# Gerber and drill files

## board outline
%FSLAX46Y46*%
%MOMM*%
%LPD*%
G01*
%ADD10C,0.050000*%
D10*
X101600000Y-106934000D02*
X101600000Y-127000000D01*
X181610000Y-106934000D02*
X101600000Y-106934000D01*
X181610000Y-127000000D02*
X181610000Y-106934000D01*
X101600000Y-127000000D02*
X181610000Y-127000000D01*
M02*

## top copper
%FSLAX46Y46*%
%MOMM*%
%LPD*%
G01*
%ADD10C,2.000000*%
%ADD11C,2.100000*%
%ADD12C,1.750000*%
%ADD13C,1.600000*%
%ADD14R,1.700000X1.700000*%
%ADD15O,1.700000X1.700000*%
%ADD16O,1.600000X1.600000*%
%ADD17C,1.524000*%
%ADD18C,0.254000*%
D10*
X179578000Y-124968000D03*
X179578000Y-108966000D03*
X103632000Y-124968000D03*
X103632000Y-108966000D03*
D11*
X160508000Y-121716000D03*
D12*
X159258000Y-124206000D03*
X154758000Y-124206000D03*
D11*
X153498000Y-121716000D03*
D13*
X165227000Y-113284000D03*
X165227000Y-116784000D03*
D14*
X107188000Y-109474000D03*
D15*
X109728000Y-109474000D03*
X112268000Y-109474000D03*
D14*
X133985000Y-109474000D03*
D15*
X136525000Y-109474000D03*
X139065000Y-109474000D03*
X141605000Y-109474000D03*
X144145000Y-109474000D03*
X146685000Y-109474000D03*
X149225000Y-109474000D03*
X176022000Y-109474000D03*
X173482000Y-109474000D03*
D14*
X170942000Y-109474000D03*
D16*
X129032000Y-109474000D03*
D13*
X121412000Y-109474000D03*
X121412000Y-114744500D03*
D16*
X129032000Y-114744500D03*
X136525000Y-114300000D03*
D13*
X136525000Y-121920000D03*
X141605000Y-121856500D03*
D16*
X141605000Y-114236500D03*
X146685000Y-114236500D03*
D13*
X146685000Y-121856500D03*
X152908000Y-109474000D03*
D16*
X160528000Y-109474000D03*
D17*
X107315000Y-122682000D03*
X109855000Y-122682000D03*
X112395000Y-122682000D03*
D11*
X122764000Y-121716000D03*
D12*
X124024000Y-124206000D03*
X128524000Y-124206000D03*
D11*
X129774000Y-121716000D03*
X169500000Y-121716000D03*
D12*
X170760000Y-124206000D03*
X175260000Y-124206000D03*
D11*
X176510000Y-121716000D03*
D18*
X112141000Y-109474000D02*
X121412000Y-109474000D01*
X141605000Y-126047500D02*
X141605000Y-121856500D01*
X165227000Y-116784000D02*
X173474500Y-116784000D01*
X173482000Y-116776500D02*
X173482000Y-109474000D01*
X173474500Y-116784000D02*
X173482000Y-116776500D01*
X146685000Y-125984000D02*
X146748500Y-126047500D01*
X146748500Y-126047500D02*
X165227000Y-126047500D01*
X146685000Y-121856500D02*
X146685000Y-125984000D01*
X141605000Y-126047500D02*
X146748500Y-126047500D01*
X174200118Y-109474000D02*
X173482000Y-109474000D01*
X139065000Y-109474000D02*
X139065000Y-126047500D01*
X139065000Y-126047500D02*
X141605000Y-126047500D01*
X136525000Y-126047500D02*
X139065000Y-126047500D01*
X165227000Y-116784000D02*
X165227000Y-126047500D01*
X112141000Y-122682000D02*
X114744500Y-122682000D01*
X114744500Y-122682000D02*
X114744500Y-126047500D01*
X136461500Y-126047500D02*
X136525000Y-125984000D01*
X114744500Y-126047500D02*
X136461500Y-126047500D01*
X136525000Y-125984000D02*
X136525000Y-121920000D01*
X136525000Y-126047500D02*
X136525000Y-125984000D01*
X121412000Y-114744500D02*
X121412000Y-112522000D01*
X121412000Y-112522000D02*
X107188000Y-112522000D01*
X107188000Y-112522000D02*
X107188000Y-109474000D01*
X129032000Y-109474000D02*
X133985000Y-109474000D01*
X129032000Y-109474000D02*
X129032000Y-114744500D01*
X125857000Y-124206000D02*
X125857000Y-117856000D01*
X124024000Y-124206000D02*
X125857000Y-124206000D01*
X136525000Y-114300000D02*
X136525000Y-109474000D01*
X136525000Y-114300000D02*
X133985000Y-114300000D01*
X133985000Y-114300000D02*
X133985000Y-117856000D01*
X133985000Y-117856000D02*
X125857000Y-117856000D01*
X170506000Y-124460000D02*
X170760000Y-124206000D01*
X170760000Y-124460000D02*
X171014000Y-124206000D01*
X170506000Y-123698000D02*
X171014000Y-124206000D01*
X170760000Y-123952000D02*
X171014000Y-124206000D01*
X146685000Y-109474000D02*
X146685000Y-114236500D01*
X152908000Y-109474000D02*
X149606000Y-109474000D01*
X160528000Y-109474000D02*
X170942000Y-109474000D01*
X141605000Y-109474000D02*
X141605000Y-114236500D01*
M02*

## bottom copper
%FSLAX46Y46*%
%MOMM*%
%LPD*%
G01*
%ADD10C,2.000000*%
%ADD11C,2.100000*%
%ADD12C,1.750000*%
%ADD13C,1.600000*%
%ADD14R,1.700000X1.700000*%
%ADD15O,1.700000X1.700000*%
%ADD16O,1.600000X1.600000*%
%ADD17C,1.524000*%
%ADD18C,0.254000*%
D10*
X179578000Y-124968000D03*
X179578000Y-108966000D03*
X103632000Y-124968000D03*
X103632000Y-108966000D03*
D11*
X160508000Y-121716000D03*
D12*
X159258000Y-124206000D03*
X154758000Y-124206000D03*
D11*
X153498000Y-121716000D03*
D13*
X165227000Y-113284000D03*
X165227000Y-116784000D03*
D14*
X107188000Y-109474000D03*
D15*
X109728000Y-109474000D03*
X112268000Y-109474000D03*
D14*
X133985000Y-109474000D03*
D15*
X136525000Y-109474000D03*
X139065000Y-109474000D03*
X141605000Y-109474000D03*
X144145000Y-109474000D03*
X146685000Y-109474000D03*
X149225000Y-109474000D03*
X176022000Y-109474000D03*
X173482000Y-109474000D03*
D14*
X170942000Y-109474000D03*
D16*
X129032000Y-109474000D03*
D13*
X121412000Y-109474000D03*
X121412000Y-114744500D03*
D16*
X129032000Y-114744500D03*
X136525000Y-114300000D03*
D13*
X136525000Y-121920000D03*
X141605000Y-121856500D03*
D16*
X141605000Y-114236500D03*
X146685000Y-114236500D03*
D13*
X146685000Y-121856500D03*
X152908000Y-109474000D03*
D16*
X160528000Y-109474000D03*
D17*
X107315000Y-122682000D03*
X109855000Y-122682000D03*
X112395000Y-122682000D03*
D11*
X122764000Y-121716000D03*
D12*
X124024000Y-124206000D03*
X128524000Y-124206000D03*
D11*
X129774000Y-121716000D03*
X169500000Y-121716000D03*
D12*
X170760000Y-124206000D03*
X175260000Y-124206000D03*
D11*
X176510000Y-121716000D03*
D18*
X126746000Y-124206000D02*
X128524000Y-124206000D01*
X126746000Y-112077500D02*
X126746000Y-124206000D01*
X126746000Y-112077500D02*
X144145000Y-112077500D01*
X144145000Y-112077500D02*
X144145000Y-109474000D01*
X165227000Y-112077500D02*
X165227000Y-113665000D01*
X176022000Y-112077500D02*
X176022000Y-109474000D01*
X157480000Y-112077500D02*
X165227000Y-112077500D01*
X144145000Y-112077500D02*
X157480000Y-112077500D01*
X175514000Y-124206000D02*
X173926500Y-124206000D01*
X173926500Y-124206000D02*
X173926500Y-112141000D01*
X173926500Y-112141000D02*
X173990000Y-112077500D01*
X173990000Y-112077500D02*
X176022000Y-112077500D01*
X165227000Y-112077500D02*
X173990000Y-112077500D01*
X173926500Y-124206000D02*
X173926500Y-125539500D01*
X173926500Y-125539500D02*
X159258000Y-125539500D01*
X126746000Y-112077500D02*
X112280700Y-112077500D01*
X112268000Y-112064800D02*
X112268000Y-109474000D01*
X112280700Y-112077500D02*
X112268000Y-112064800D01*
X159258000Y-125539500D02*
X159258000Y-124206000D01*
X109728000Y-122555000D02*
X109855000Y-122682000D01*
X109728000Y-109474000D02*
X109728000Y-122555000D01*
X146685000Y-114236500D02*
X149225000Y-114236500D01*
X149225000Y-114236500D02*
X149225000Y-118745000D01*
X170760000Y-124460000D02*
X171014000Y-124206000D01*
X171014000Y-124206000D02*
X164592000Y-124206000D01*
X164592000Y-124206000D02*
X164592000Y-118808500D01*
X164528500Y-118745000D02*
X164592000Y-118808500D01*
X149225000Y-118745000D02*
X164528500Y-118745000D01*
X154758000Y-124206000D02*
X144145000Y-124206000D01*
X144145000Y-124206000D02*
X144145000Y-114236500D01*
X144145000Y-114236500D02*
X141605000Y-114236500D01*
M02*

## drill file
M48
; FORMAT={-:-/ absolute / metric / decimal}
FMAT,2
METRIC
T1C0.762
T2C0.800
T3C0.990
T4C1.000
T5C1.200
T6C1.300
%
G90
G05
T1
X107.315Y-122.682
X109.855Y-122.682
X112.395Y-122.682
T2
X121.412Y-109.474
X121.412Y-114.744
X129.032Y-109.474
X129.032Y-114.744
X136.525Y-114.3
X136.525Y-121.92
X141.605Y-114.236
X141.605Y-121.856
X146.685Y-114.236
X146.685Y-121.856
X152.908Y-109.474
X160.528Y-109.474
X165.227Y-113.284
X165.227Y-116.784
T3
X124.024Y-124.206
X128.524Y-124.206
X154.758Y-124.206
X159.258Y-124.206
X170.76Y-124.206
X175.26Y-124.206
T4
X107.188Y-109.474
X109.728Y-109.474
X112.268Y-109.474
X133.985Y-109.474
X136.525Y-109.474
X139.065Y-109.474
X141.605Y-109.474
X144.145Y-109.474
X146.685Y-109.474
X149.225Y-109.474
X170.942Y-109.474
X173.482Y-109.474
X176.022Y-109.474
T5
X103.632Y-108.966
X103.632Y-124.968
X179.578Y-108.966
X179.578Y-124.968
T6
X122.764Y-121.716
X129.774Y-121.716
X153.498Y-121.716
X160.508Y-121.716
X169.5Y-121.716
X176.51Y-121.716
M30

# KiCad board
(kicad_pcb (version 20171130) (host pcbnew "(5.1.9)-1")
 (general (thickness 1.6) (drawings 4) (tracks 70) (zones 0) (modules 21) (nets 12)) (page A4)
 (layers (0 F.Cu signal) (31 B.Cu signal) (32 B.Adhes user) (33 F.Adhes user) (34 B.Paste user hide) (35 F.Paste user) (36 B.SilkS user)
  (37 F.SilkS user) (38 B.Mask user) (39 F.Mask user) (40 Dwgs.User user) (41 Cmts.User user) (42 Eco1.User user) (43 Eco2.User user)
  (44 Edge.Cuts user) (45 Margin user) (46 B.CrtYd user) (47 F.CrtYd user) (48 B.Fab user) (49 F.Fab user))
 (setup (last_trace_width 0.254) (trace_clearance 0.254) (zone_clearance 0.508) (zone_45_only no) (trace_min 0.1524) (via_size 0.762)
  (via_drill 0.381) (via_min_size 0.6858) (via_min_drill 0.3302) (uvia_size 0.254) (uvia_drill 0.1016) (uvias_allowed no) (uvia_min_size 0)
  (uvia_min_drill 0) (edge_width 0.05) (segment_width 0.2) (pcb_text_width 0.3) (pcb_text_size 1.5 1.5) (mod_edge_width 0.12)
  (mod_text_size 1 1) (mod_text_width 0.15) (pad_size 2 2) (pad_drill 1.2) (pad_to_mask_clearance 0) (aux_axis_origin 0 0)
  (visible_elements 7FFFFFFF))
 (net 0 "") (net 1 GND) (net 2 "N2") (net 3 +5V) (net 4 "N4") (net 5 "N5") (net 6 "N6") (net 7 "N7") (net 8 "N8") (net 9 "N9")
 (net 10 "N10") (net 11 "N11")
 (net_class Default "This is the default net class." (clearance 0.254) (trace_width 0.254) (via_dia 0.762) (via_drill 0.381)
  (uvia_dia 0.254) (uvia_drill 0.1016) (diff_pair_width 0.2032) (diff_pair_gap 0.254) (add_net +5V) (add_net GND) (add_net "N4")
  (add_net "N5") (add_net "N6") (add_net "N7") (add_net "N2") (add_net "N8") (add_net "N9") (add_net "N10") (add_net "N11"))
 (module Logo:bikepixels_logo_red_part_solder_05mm (layer F.Cu) (at 106.553 116.4463)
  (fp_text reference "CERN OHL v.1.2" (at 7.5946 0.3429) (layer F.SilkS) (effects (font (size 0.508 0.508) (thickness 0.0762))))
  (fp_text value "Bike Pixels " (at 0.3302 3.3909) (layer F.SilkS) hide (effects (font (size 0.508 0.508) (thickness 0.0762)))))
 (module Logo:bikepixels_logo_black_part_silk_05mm (layer F.Cu) (at 106.553 115.7732)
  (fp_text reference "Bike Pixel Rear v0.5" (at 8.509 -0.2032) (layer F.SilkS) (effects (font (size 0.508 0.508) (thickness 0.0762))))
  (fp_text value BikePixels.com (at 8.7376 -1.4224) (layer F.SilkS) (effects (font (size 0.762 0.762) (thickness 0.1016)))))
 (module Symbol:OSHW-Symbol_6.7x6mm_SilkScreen (layer F.Cu) (at 177.8 115.57)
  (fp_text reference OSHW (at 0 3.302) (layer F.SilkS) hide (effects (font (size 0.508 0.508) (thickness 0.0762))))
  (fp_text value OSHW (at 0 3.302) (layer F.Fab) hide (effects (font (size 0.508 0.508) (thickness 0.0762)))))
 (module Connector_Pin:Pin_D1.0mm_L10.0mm (layer F.Cu) (at 179.578 124.968)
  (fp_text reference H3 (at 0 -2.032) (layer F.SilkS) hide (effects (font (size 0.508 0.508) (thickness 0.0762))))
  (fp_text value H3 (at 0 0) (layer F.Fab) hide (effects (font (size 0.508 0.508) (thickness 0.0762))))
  (pad "" thru_hole circle (at 0 0) (size 2 2) (drill 1.2) (layers *.Cu *.Mask)))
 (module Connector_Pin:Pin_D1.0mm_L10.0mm (layer F.Cu) (at 179.578 108.966)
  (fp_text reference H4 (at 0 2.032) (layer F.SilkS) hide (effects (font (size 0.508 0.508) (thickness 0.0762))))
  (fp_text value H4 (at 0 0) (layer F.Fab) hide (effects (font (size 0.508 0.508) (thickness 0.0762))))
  (pad "" thru_hole circle (at 0 0) (size 2 2) (drill 1.2) (layers *.Cu *.Mask)))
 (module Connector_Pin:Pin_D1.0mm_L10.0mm (layer F.Cu) (at 103.632 124.968)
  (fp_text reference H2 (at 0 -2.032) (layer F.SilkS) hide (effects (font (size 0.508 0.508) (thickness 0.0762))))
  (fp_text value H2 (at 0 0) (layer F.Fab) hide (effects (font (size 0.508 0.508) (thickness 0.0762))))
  (pad "" thru_hole circle (at 0 0) (size 2 2) (drill 1.2) (layers *.Cu *.Mask)))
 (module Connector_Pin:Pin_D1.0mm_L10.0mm (layer F.Cu) (at 103.632 108.966)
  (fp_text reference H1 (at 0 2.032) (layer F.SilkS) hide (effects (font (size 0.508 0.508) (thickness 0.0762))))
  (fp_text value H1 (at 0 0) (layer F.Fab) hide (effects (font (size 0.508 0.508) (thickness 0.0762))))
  (pad "" thru_hole circle (at 0 0) (size 2 2) (drill 1.2) (layers *.Cu *.Mask)))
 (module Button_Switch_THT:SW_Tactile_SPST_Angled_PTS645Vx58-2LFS (layer F.Cu) (at 159.258 124.206 180)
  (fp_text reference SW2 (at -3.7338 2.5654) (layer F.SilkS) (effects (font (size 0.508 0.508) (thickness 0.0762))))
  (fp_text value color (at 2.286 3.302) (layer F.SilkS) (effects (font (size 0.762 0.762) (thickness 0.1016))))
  (pad "" thru_hole circle (at -1.25 2.49 180) (size 2.1 2.1) (drill 1.3) (layers *.Cu *.Mask))
  (pad 1 thru_hole circle (at 0 0 180) (size 1.75 1.75) (drill 0.99) (layers *.Cu *.Mask) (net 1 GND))
  (pad 2 thru_hole circle (at 4.5 0 180) (size 1.75 1.75) (drill 0.99) (layers *.Cu *.Mask) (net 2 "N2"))
  (pad "" thru_hole circle (at 5.76 2.49 180) (size 2.1 2.1) (drill 1.3) (layers *.Cu *.Mask)))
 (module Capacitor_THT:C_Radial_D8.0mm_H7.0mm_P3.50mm (layer F.Cu) (at 165.227 113.284 270)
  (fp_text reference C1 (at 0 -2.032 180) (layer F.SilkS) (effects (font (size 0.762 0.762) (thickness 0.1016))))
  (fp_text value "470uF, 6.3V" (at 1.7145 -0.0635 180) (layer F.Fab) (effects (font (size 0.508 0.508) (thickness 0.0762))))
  (pad 1 thru_hole circle (at 0 0 270) (size 1.6 1.6) (drill 0.8) (layers *.Cu *.Mask) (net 1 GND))
  (pad 2 thru_hole circle (at 3.5 0 270) (size 1.6 1.6) (drill 0.8) (layers *.Cu *.Mask) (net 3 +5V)))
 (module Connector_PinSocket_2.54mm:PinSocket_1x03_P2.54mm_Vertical (layer F.Cu) (at 107.188 109.474 90)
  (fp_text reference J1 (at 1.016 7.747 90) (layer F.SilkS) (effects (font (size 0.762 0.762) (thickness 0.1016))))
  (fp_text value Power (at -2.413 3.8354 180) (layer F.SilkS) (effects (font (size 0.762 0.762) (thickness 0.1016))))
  (pad 1 thru_hole rect (at 0 0 90) (size 1.7 1.7) (drill 1) (layers *.Cu *.Mask) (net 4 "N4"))
  (pad 2 thru_hole oval (at 0 2.54 90) (size 1.7 1.7) (drill 1) (layers *.Cu *.Mask) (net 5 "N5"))
  (pad 3 thru_hole oval (at 0 5.08 90) (size 1.7 1.7) (drill 1) (layers *.Cu *.Mask) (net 1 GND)))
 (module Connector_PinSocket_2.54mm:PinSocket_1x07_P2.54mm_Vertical (layer F.Cu) (at 133.985 109.474 90)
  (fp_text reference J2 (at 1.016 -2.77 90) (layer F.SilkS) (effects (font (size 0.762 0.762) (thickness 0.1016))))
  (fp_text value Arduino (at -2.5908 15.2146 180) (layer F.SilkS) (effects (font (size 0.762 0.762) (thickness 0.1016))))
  (pad 1 thru_hole rect (at 0 0 90) (size 1.7 1.7) (drill 1) (layers *.Cu *.Mask) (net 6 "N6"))
  (pad 2 thru_hole oval (at 0 2.54 90) (size 1.7 1.7) (drill 1) (layers *.Cu *.Mask) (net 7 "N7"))
  (pad 3 thru_hole oval (at 0 5.08 90) (size 1.7 1.7) (drill 1) (layers *.Cu *.Mask) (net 3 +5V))
  (pad 4 thru_hole oval (at 0 7.62 90) (size 1.7 1.7) (drill 1) (layers *.Cu *.Mask) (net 2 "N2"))
  (pad 5 thru_hole oval (at 0 10.16 90) (size 1.7 1.7) (drill 1) (layers *.Cu *.Mask) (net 1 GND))
  (pad 6 thru_hole oval (at 0 12.7 90) (size 1.7 1.7) (drill 1) (layers *.Cu *.Mask) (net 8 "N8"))
  (pad 7 thru_hole oval (at 0 15.24 90) (size 1.7 1.7) (drill 1) (layers *.Cu *.Mask) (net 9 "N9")))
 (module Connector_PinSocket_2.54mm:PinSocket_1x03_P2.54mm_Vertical (layer F.Cu) (at 170.942 109.474 90)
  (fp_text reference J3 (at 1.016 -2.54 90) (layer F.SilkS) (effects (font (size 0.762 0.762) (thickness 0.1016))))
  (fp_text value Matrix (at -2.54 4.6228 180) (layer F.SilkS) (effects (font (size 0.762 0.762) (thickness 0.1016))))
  (pad 3 thru_hole oval (at 0 5.08 90) (size 1.7 1.7) (drill 1) (layers *.Cu *.Mask) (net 1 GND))
  (pad 2 thru_hole oval (at 0 2.54 90) (size 1.7 1.7) (drill 1) (layers *.Cu *.Mask) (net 3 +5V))
  (pad 1 thru_hole rect (at 0 0 90) (size 1.7 1.7) (drill 1) (layers *.Cu *.Mask) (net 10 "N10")))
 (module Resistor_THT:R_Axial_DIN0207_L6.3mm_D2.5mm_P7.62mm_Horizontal (layer F.Cu) (at 121.412 109.474)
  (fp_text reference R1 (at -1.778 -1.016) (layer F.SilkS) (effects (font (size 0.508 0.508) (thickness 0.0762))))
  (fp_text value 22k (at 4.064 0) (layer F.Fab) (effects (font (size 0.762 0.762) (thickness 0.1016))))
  (pad 2 thru_hole oval (at 7.62 0) (size 1.6 1.6) (drill 0.8) (layers *.Cu *.Mask) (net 6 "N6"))
  (pad 1 thru_hole circle (at 0 0) (size 1.6 1.6) (drill 0.8) (layers *.Cu *.Mask) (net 1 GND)))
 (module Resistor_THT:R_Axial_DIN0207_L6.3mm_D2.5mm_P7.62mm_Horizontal (layer F.Cu) (at 121.412 114.7445)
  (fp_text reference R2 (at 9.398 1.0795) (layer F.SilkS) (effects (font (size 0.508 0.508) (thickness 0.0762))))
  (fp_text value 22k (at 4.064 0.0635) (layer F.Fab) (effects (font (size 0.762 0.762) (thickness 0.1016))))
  (pad 1 thru_hole circle (at 0 0) (size 1.6 1.6) (drill 0.8) (layers *.Cu *.Mask) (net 4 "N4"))
  (pad 2 thru_hole oval (at 7.62 0) (size 1.6 1.6) (drill 0.8) (layers *.Cu *.Mask) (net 6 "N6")))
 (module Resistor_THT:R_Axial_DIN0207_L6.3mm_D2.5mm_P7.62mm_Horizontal (layer F.Cu) (at 136.525 121.92 90)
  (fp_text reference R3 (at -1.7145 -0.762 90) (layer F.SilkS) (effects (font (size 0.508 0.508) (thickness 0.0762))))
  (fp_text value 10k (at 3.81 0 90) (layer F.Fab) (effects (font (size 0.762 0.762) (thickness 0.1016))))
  (pad 2 thru_hole oval (at 7.62 0 90) (size 1.6 1.6) (drill 0.8) (layers *.Cu *.Mask) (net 7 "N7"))
  (pad 1 thru_hole circle (at 0 0 90) (size 1.6 1.6) (drill 0.8) (layers *.Cu *.Mask) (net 3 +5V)))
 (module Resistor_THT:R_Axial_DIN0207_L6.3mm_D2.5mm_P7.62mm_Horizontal (layer F.Cu) (at 141.605 121.8565 90)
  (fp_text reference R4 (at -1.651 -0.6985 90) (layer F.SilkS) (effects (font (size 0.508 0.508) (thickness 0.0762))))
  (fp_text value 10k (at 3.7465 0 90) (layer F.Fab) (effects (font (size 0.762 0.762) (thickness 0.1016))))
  (pad 1 thru_hole circle (at 0 0 90) (size 1.6 1.6) (drill 0.8) (layers *.Cu *.Mask) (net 3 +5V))
  (pad 2 thru_hole oval (at 7.62 0 90) (size 1.6 1.6) (drill 0.8) (layers *.Cu *.Mask) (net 2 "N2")))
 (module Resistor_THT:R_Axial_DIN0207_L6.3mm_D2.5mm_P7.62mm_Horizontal (layer F.Cu) (at 146.685 121.8565 90)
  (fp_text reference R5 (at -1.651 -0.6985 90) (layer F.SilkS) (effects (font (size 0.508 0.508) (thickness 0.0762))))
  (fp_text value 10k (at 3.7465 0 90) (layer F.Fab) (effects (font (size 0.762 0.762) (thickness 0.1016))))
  (pad 2 thru_hole oval (at 7.62 0 90) (size 1.6 1.6) (drill 0.8) (layers *.Cu *.Mask) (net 8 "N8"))
  (pad 1 thru_hole circle (at 0 0 90) (size 1.6 1.6) (drill 0.8) (layers *.Cu *.Mask) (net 3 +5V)))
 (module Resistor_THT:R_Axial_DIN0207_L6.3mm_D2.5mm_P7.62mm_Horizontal (layer F.Cu) (at 152.908 109.474)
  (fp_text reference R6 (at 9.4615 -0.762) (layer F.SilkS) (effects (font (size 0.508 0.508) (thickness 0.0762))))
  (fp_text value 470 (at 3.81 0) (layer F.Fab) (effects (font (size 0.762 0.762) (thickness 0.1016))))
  (pad 1 thru_hole circle (at 0 0) (size 1.6 1.6) (drill 0.8) (layers *.Cu *.Mask) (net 9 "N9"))
  (pad 2 thru_hole oval (at 7.62 0) (size 1.6 1.6) (drill 0.8) (layers *.Cu *.Mask) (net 10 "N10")))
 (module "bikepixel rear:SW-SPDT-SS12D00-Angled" (layer F.Cu) (at 109.855 122.682)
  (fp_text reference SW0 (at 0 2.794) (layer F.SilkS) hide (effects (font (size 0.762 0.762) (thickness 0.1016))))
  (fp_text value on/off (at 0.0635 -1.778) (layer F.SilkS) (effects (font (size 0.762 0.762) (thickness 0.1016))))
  (pad 1 thru_hole circle (at -2.54 0) (size 1.524 1.524) (drill 0.762) (layers *.Cu *.Mask) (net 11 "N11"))
  (pad 2 thru_hole circle (at 0 0) (size 1.524 1.524) (drill 0.762) (layers *.Cu *.Mask) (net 5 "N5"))
  (pad 3 thru_hole circle (at 2.54 0) (size 1.524 1.524) (drill 0.762) (layers *.Cu *.Mask) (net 3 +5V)))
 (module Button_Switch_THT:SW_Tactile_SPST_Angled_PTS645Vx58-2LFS (layer F.Cu) (at 128.524 124.206 180)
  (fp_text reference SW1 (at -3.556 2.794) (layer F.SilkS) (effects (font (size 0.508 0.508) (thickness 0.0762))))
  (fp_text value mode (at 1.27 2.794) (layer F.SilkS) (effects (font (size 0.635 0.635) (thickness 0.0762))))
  (pad "" thru_hole circle (at 5.76 2.49 180) (size 2.1 2.1) (drill 1.3) (layers *.Cu *.Mask))
  (pad 2 thru_hole circle (at 4.5 0 180) (size 1.75 1.75) (drill 0.99) (layers *.Cu *.Mask) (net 7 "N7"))
  (pad 1 thru_hole circle (at 0 0 180) (size 1.75 1.75) (drill 0.99) (layers *.Cu *.Mask) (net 1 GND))
  (pad "" thru_hole circle (at -1.25 2.49 180) (size 2.1 2.1) (drill 1.3) (layers *.Cu *.Mask)))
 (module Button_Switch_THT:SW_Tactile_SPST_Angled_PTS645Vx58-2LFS (layer F.Cu) (at 175.26 124.206 180)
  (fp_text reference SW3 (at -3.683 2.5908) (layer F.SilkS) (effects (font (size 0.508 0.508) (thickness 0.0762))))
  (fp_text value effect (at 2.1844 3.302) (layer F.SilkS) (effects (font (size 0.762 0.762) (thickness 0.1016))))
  (pad "" thru_hole circle (at 5.76 2.49 180) (size 2.1 2.1) (drill 1.3) (layers *.Cu *.Mask))
  (pad 2 thru_hole circle (at 4.5 0 180) (size 1.75 1.75) (drill 0.99) (layers *.Cu *.Mask) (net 8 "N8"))
  (pad 1 thru_hole circle (at 0 0 180) (size 1.75 1.75) (drill 0.99) (layers *.Cu *.Mask) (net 1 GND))
  (pad "" thru_hole circle (at -1.25 2.49 180) (size 2.1 2.1) (drill 1.3) (layers *.Cu *.Mask)))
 (gr_line (start 101.6 106.934) (end 101.6 127) (layer Edge.Cuts) (width 0.05))
 (gr_line (start 181.61 106.934) (end 101.6 106.934) (layer Edge.Cuts) (width 0.05))
 (gr_line (start 181.61 127) (end 181.61 106.934) (layer Edge.Cuts) (width 0.05))
 (gr_line (start 101.6 127) (end 181.61 127) (layer Edge.Cuts) (width 0.05))
 (segment (start 112.141 109.474) (end 121.412 109.474) (width 0.254) (layer F.Cu) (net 1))
 (segment (start 126.746 124.206) (end 128.524 124.206) (width 0.254) (layer B.Cu) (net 1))
 (segment (start 126.746 112.0775) (end 126.746 124.206) (width 0.254) (layer B.Cu) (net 1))
 (segment (start 126.746 112.0775) (end 144.145 112.0775) (width 0.254) (layer B.Cu) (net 1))
 (segment (start 144.145 112.0775) (end 144.145 109.474) (width 0.254) (layer B.Cu) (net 1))
 (segment (start 165.227 112.0775) (end 165.227 113.665) (width 0.254) (layer B.Cu) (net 1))
 (segment (start 176.022 112.0775) (end 176.022 109.474) (width 0.254) (layer B.Cu) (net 1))
 (segment (start 157.48 112.0775) (end 165.227 112.0775) (width 0.254) (layer B.Cu) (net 1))
 (segment (start 144.145 112.0775) (end 157.48 112.0775) (width 0.254) (layer B.Cu) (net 1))
 (segment (start 175.514 124.206) (end 173.9265 124.206) (width 0.254) (layer B.Cu) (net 1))
 (segment (start 173.9265 124.206) (end 173.9265 112.141) (width 0.254) (layer B.Cu) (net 1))
 (segment (start 173.9265 112.141) (end 173.99 112.0775) (width 0.254) (layer B.Cu) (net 1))
 (segment (start 173.99 112.0775) (end 176.022 112.0775) (width 0.254) (layer B.Cu) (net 1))
 (segment (start 165.227 112.0775) (end 173.99 112.0775) (width 0.254) (layer B.Cu) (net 1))
 (segment (start 173.9265 124.206) (end 173.9265 125.5395) (width 0.254) (layer B.Cu) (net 1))
 (segment (start 173.9265 125.5395) (end 159.258 125.5395) (width 0.254) (layer B.Cu) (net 1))
 (segment (start 126.746 112.0775) (end 112.2807 112.0775) (width 0.254) (layer B.Cu) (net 1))
 (segment (start 112.268 112.0648) (end 112.268 109.474) (width 0.254) (layer B.Cu) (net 1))
 (segment (start 112.2807 112.0775) (end 112.268 112.0648) (width 0.254) (layer B.Cu) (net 1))
 (segment (start 159.258 125.5395) (end 159.258 124.206) (width 0.254) (layer B.Cu) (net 1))
 (segment (start 141.605 126.0475) (end 141.605 121.8565) (width 0.254) (layer F.Cu) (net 3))
 (segment (start 165.227 116.784) (end 173.4745 116.784) (width 0.254) (layer F.Cu) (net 3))
 (segment (start 173.482 116.7765) (end 173.482 109.474) (width 0.254) (layer F.Cu) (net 3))
 (segment (start 173.4745 116.784) (end 173.482 116.7765) (width 0.254) (layer F.Cu) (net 3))
 (segment (start 146.685 125.984) (end 146.7485 126.0475) (width 0.254) (layer F.Cu) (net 3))
 (segment (start 146.7485 126.0475) (end 165.227 126.0475) (width 0.254) (layer F.Cu) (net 3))
 (segment (start 146.685 121.8565) (end 146.685 125.984) (width 0.254) (layer F.Cu) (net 3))
 (segment (start 141.605 126.0475) (end 146.7485 126.0475) (width 0.254) (layer F.Cu) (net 3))
 (segment (start 174.200118 109.474) (end 173.482 109.474) (width 0.254) (layer F.Cu) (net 3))
 (segment (start 139.065 109.474) (end 139.065 126.0475) (width 0.254) (layer F.Cu) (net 3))
 (segment (start 139.065 126.0475) (end 141.605 126.0475) (width 0.254) (layer F.Cu) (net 3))
 (segment (start 136.525 126.0475) (end 139.065 126.0475) (width 0.254) (layer F.Cu) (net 3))
 (segment (start 165.227 116.784) (end 165.227 126.0475) (width 0.254) (layer F.Cu) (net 3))
 (segment (start 112.141 122.682) (end 114.7445 122.682) (width 0.254) (layer F.Cu) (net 3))
 (segment (start 114.7445 122.682) (end 114.7445 126.0475) (width 0.254) (layer F.Cu) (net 3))
 (segment (start 136.4615 126.0475) (end 136.525 125.984) (width 0.254) (layer F.Cu) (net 3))
 (segment (start 114.7445 126.0475) (end 136.4615 126.0475) (width 0.254) (layer F.Cu) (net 3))
 (segment (start 136.525 125.984) (end 136.525 121.92) (width 0.254) (layer F.Cu) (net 3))
 (segment (start 136.525 126.0475) (end 136.525 125.984) (width 0.254) (layer F.Cu) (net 3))
 (segment (start 121.412 114.7445) (end 121.412 112.522) (width 0.254) (layer F.Cu) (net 4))
 (segment (start 121.412 112.522) (end 107.188 112.522) (width 0.254) (layer F.Cu) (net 4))
 (segment (start 107.188 112.522) (end 107.188 109.474) (width 0.254) (layer F.Cu) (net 4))
 (segment (start 109.728 122.555) (end 109.855 122.682) (width 0.254) (layer B.Cu) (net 5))
 (segment (start 109.728 109.474) (end 109.728 122.555) (width 0.254) (layer B.Cu) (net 5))
 (segment (start 129.032 109.474) (end 133.985 109.474) (width 0.254) (layer F.Cu) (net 6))
 (segment (start 129.032 109.474) (end 129.032 114.7445) (width 0.254) (layer F.Cu) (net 6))
 (segment (start 125.857 124.206) (end 125.857 117.856) (width 0.254) (layer F.Cu) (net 7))
 (segment (start 124.024 124.206) (end 125.857 124.206) (width 0.254) (layer F.Cu) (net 7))
 (segment (start 136.525 114.3) (end 136.525 109.474) (width 0.254) (layer F.Cu) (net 7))
 (segment (start 136.525 114.3) (end 133.985 114.3) (width 0.254) (layer F.Cu) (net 7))
 (segment (start 133.985 114.3) (end 133.985 117.856) (width 0.254) (layer F.Cu) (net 7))
 (segment (start 133.985 117.856) (end 125.857 117.856) (width 0.254) (layer F.Cu) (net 7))
 (segment (start 170.506 124.46) (end 170.76 124.206) (width 0.254) (layer F.Cu) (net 8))
 (segment (start 170.76 124.46) (end 171.014 124.206) (width 0.254) (layer F.Cu) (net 8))
 (segment (start 170.506 123.698) (end 171.014 124.206) (width 0.254) (layer F.Cu) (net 8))
 (segment (start 170.76 123.952) (end 171.014 124.206) (width 0.254) (layer F.Cu) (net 8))
 (segment (start 146.685 109.474) (end 146.685 114.2365) (width 0.254) (layer F.Cu) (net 8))
 (segment (start 146.685 114.2365) (end 149.225 114.2365) (width 0.254) (layer B.Cu) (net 8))
 (segment (start 149.225 114.2365) (end 149.225 118.745) (width 0.254) (layer B.Cu) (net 8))
 (segment (start 170.76 124.46) (end 171.014 124.206) (width 0.254) (layer B.Cu) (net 8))
 (segment (start 171.014 124.206) (end 164.592 124.206) (width 0.254) (layer B.Cu) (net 8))
 (segment (start 164.592 124.206) (end 164.592 118.8085) (width 0.254) (layer B.Cu) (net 8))
 (segment (start 164.5285 118.745) (end 164.592 118.8085) (width 0.254) (layer B.Cu) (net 8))
 (segment (start 149.225 118.745) (end 164.5285 118.745) (width 0.254) (layer B.Cu) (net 8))
 (segment (start 152.908 109.474) (end 149.606 109.474) (width 0.254) (layer F.Cu) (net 9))
 (segment (start 160.528 109.474) (end 170.942 109.474) (width 0.254) (layer F.Cu) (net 10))
 (segment (start 141.605 109.474) (end 141.605 114.2365) (width 0.254) (layer F.Cu) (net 2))
 (segment (start 154.758 124.206) (end 144.145 124.206) (width 0.254) (layer B.Cu) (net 2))
 (segment (start 144.145 124.206) (end 144.145 114.2365) (width 0.254) (layer B.Cu) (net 2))
 (segment (start 144.145 114.2365) (end 141.605 114.2365) (width 0.254) (layer B.Cu) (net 2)))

